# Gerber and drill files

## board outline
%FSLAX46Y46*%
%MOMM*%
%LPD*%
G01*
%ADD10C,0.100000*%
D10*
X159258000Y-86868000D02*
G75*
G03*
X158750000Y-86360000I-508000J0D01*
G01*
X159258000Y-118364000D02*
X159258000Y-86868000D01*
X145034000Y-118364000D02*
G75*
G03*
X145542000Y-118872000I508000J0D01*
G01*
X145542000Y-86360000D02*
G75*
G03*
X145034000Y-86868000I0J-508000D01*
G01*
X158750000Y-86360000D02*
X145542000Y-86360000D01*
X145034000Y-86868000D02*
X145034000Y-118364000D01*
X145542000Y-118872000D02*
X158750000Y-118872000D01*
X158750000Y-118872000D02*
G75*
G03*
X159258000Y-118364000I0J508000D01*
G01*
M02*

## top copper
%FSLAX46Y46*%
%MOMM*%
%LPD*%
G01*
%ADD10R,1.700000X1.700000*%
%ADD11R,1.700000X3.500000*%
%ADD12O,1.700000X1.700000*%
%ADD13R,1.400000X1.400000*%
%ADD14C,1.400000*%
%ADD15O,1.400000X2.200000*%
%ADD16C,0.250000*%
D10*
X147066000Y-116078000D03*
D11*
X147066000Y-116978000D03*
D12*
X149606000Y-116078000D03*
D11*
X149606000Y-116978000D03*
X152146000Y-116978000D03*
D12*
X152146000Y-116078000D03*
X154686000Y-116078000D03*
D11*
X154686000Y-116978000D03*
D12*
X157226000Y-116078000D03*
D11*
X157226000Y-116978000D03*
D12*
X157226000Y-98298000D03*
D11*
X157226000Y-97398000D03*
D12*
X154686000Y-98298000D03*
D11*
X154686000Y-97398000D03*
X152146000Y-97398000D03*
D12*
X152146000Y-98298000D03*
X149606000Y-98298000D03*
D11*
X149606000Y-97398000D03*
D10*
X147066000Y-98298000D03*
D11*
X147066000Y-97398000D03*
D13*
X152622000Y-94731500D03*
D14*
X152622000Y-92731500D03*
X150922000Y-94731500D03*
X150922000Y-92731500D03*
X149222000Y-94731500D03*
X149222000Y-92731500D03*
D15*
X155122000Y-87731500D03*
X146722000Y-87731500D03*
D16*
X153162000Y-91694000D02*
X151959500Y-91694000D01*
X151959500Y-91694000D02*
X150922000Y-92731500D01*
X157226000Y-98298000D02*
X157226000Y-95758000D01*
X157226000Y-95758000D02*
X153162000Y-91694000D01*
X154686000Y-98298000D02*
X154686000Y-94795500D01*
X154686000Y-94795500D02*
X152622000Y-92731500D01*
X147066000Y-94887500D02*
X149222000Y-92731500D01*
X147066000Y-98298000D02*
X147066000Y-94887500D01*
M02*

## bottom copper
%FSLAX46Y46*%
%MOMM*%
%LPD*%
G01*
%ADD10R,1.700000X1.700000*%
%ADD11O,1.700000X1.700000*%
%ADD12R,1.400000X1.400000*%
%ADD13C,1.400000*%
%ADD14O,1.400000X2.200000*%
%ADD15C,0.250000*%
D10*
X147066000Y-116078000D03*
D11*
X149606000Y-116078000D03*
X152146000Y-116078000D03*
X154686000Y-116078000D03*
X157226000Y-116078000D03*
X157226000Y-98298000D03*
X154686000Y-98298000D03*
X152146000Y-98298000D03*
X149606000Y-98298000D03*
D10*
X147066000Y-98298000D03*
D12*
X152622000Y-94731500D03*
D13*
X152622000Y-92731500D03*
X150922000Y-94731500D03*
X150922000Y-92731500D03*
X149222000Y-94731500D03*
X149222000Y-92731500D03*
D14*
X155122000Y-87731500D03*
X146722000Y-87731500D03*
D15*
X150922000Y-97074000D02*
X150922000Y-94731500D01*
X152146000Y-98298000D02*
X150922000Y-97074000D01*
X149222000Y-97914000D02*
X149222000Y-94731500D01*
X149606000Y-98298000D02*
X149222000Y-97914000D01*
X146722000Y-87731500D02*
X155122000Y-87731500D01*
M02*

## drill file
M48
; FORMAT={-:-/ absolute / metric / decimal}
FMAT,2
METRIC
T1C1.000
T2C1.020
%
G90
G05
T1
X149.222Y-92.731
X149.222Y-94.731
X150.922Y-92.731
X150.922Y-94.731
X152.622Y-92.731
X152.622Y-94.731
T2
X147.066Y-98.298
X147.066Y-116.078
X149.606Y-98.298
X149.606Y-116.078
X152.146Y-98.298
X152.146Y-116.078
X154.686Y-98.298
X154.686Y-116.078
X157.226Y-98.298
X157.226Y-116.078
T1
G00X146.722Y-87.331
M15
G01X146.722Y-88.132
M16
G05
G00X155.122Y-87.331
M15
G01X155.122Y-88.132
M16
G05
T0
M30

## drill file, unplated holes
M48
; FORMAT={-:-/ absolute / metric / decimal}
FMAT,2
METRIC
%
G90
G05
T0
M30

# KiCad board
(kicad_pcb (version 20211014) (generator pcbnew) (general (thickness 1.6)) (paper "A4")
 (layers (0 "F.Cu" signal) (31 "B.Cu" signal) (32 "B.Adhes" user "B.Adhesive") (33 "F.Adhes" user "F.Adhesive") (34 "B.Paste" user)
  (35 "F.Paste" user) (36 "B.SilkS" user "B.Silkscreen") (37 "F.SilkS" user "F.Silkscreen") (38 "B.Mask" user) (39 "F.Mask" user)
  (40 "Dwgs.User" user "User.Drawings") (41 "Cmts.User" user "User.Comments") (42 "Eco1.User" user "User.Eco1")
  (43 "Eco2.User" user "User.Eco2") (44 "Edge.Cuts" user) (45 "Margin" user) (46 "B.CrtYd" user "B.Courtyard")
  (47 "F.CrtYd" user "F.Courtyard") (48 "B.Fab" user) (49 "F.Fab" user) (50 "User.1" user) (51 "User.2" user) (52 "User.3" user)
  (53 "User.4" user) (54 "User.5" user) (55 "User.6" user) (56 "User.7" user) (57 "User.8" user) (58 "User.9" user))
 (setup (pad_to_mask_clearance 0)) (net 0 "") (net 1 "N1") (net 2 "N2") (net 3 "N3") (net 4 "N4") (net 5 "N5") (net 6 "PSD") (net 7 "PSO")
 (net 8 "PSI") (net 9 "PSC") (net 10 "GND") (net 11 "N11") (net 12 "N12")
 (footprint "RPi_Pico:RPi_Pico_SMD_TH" (layer "F.Cu") (at 152.146 107.188 90)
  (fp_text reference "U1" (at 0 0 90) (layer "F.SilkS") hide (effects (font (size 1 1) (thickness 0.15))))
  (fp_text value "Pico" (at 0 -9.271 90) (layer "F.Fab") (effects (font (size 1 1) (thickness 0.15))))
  (pad "13" thru_hole rect (at -8.89 -5.08 90) (size 1.7 1.7) (drill 1.02) (layers *.Cu *.Mask) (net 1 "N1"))
  (pad "13" smd rect (at -8.89 -5.08 90) (size 3.5 1.7) (drill (offset -0.9 0)) (layers "F.Cu" "F.Mask") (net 1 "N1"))
  (pad "14" thru_hole oval (at -8.89 -2.54 90) (size 1.7 1.7) (drill 1.02) (layers *.Cu *.Mask) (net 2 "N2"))
  (pad "14" smd rect (at -8.89 -2.54 90) (size 3.5 1.7) (drill (offset -0.9 0)) (layers "F.Cu" "F.Mask") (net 2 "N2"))
  (pad "15" smd rect (at -8.89 0 90) (size 3.5 1.7) (drill (offset -0.9 0)) (layers "F.Cu" "F.Mask") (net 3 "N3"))
  (pad "15" thru_hole oval (at -8.89 0 90) (size 1.7 1.7) (drill 1.02) (layers *.Cu *.Mask) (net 3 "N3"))
  (pad "16" thru_hole oval (at -8.89 2.54 90) (size 1.7 1.7) (drill 1.02) (layers *.Cu *.Mask) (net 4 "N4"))
  (pad "16" smd rect (at -8.89 2.54 90) (size 3.5 1.7) (drill (offset -0.9 0)) (layers "F.Cu" "F.Mask") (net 4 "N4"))
  (pad "17" thru_hole oval (at -8.89 5.08 90) (size 1.7 1.7) (drill 1.02) (layers *.Cu *.Mask) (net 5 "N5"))
  (pad "17" smd rect (at -8.89 5.08 90) (size 3.5 1.7) (drill (offset -0.9 0)) (layers "F.Cu" "F.Mask") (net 5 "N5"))
  (pad "24" thru_hole oval (at 8.89 5.08 90) (size 1.7 1.7) (drill 1.02) (layers *.Cu *.Mask) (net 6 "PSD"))
  (pad "24" smd rect (at 8.89 5.08 90) (size 3.5 1.7) (drill (offset 0.9 0)) (layers "F.Cu" "F.Mask") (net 6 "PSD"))
  (pad "25" thru_hole oval (at 8.89 2.54 90) (size 1.7 1.7) (drill 1.02) (layers *.Cu *.Mask) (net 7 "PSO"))
  (pad "25" smd rect (at 8.89 2.54 90) (size 3.5 1.7) (drill (offset 0.9 0)) (layers "F.Cu" "F.Mask") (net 7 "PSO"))
  (pad "26" smd rect (at 8.89 0 90) (size 3.5 1.7) (drill (offset 0.9 0)) (layers "F.Cu" "F.Mask") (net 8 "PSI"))
  (pad "26" thru_hole oval (at 8.89 0 90) (size 1.7 1.7) (drill 1.02) (layers *.Cu *.Mask) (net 8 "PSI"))
  (pad "27" thru_hole oval (at 8.89 -2.54 90) (size 1.7 1.7) (drill 1.02) (layers *.Cu *.Mask) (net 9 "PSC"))
  (pad "27" smd rect (at 8.89 -2.54 90) (size 3.5 1.7) (drill (offset 0.9 0)) (layers "F.Cu" "F.Mask") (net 9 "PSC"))
  (pad "28" thru_hole rect (at 8.89 -5.08 90) (size 1.7 1.7) (drill 1.02) (layers *.Cu *.Mask) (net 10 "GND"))
  (pad "28" smd rect (at 8.89 -5.08 90) (size 3.5 1.7) (drill (offset 0.9 0)) (layers "F.Cu" "F.Mask") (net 10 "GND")))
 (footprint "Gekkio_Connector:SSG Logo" (layer "B.Cu") (at 152.146 103.886 180)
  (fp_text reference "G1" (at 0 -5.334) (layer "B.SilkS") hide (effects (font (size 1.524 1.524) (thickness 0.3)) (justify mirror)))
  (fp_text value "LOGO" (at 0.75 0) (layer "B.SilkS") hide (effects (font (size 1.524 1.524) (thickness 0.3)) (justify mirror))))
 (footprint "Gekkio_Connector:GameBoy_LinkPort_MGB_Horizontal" (layer "B.Cu") (at 152.742 95.3515 90)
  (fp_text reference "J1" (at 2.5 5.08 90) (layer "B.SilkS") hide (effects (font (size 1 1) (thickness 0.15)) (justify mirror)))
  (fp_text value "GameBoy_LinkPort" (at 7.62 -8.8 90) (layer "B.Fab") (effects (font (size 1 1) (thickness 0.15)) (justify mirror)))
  (pad "1" thru_hole rect (at 0.62 -0.12 90) (size 1.4 1.4) (drill 1) (layers *.Cu *.Mask) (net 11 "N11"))
  (pad "2" thru_hole circle (at 2.62 -0.12 90) (size 1.4 1.4) (drill 1) (layers *.Cu *.Mask) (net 7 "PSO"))
  (pad "3" thru_hole circle (at 0.62 -1.82 90) (size 1.4 1.4) (drill 1) (layers *.Cu *.Mask) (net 8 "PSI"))
  (pad "4" thru_hole circle (at 2.62 -1.82 90) (size 1.4 1.4) (drill 1) (layers *.Cu *.Mask) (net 6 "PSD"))
  (pad "5" thru_hole circle (at 0.62 -3.52 90) (size 1.4 1.4) (drill 1) (layers *.Cu *.Mask) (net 9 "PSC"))
  (pad "6" thru_hole circle (at 2.62 -3.52 90) (size 1.4 1.4) (drill 1) (layers *.Cu *.Mask) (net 10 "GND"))
  (pad "SH" thru_hole oval (at 7.62 2.38) (size 1.4 2.2) (drill oval 1 1.8) (layers *.Cu *.Mask) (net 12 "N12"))
  (pad "SH" thru_hole oval (at 7.62 -6.02) (size 1.4 2.2) (drill oval 1 1.8) (layers *.Cu *.Mask) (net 12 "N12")))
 (gr_arc (start 158.75 86.36) (mid 159.10921 86.50879) (end 159.258 86.868) (layer "Edge.Cuts") (width 0.1))
 (gr_line (start 159.258 118.364) (end 159.258 86.868) (layer "Edge.Cuts") (width 0.1))
 (gr_arc (start 145.542 118.872) (mid 145.18279 118.72321) (end 145.034 118.364) (layer "Edge.Cuts") (width 0.1))
 (gr_arc (start 145.034 86.868) (mid 145.18279 86.50879) (end 145.542 86.36) (layer "Edge.Cuts") (width 0.1))
 (gr_line (start 158.75 86.36) (end 145.542 86.36) (layer "Edge.Cuts") (width 0.1))
 (gr_line (start 145.034 86.868) (end 145.034 118.364) (layer "Edge.Cuts") (width 0.1))
 (gr_line (start 145.542 118.872) (end 158.75 118.872) (layer "Edge.Cuts") (width 0.1))
 (gr_arc (start 159.258 118.364) (mid 159.10921 118.72321) (end 158.75 118.872) (layer "Edge.Cuts") (width 0.1))
 (segment (start 150.922 97.074) (end 150.922 94.7315) (width 0.25) (layer "B.Cu") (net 8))
 (segment (start 152.146 98.298) (end 150.922 97.074) (width 0.25) (layer "B.Cu") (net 8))
 (segment (start 153.162 91.694) (end 151.9595 91.694) (width 0.25) (layer "F.Cu") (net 6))
 (segment (start 151.9595 91.694) (end 150.922 92.7315) (width 0.25) (layer "F.Cu") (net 6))
 (segment (start 157.226 98.298) (end 157.226 95.758) (width 0.25) (layer "F.Cu") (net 6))
 (segment (start 157.226 95.758) (end 153.162 91.694) (width 0.25) (layer "F.Cu") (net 6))
 (segment (start 149.222 97.914) (end 149.222 94.7315) (width 0.25) (layer "B.Cu") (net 9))
 (segment (start 149.606 98.298) (end 149.222 97.914) (width 0.25) (layer "B.Cu") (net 9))
 (segment (start 154.686 98.298) (end 154.686 94.7955) (width 0.25) (layer "F.Cu") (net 7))
 (segment (start 154.686 94.7955) (end 152.622 92.7315) (width 0.25) (layer "F.Cu") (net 7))
 (segment (start 147.066 94.8875) (end 149.222 92.7315) (width 0.25) (layer "F.Cu") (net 10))
 (segment (start 147.066 98.298) (end 147.066 94.8875) (width 0.25) (layer "F.Cu") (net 10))
 (segment (start 146.722 87.7315) (end 155.122 87.7315) (width 0.25) (layer "B.Cu") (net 12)))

